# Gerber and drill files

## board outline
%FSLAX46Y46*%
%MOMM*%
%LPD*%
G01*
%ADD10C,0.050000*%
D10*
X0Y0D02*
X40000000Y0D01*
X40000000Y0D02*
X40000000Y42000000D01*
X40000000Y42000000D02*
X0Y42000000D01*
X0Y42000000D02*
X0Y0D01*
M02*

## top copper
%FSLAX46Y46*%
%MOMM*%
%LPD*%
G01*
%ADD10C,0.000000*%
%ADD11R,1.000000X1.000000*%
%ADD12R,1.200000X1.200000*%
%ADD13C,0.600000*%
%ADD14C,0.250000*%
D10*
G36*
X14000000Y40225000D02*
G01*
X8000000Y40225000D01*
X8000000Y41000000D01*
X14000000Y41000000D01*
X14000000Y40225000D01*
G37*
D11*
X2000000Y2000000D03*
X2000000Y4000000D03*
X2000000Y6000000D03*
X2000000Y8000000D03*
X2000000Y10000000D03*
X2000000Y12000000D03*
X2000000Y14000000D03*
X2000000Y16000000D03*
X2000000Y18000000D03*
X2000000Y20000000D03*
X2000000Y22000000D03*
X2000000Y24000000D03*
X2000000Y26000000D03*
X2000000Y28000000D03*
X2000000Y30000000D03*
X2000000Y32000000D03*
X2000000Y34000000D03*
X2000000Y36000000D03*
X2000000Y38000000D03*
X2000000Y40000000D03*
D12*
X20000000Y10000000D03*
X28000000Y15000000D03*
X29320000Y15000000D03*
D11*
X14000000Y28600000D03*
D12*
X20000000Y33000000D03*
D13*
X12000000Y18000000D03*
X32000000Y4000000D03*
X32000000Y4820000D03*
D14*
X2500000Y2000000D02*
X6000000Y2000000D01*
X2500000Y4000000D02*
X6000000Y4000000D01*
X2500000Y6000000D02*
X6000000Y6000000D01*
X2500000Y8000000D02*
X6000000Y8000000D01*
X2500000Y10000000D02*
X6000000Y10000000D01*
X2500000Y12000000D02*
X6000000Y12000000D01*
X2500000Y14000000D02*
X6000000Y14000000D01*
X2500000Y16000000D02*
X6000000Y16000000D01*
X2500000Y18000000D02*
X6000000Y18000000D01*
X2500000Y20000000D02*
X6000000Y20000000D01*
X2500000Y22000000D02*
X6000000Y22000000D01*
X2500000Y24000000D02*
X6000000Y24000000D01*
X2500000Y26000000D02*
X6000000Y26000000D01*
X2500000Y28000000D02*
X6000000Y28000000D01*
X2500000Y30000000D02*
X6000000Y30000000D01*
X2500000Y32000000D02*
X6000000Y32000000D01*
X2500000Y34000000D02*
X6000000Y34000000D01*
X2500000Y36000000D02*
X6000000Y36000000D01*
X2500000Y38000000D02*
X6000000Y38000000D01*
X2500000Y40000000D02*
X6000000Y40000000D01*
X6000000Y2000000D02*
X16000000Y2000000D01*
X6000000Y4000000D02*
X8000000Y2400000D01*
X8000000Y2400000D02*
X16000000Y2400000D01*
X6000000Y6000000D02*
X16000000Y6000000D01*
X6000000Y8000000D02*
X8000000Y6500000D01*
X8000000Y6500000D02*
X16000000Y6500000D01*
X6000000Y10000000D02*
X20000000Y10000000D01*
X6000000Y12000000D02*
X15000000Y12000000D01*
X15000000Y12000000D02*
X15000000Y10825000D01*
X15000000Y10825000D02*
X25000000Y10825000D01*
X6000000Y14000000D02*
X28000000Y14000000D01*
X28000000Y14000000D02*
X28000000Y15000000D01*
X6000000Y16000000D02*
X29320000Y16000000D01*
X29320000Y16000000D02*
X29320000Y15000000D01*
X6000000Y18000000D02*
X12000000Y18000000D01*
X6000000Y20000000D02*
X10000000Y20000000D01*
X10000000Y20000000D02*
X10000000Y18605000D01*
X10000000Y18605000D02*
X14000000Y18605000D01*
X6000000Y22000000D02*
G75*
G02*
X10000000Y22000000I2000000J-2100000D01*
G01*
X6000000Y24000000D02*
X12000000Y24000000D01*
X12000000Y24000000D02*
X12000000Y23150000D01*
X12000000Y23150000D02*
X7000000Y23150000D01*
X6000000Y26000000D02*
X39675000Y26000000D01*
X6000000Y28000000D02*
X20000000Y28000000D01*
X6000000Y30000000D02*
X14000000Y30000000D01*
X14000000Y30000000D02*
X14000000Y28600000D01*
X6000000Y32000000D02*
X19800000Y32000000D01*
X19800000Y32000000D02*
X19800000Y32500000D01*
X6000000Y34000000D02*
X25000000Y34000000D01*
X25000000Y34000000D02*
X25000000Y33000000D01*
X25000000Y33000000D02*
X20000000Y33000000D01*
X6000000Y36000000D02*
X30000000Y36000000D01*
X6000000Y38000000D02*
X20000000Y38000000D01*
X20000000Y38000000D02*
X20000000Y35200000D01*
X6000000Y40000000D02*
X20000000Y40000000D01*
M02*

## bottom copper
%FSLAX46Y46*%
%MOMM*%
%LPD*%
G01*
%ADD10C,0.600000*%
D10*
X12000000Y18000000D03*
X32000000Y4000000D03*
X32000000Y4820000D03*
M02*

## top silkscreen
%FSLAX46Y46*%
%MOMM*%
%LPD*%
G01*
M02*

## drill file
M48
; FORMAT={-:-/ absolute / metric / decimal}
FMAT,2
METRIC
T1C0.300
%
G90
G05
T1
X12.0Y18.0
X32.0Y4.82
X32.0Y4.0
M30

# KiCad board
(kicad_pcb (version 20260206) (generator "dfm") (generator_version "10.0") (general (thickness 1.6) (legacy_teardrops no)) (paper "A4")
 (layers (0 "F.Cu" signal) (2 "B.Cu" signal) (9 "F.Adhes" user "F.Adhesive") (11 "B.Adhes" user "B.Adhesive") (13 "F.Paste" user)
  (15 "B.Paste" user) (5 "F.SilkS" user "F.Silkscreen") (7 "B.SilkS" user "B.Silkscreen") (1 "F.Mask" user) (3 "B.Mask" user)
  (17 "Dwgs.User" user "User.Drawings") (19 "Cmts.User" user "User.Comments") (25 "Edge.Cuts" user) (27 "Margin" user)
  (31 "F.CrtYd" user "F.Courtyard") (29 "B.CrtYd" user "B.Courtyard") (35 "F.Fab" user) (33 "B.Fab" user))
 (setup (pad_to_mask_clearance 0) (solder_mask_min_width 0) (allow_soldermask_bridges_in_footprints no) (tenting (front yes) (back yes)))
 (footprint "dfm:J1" (layer "F.Cu") (at 2 -21 0)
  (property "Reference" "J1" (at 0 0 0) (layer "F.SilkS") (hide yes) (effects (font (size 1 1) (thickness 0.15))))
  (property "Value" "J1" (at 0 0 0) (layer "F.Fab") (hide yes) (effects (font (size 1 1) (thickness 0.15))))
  (pad "1" smd rect (at 0 19 0) (size 1 1) (layers "F.Cu" "F.Mask" "F.Paste") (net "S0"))
  (pad "2" smd rect (at 0 17 0) (size 1 1) (layers "F.Cu" "F.Mask" "F.Paste") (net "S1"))
  (pad "3" smd rect (at 0 15 0) (size 1 1) (layers "F.Cu" "F.Mask" "F.Paste") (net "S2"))
  (pad "4" smd rect (at 0 13 0) (size 1 1) (layers "F.Cu" "F.Mask" "F.Paste") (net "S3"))
  (pad "5" smd rect (at 0 11 0) (size 1 1) (layers "F.Cu" "F.Mask" "F.Paste") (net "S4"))
  (pad "6" smd rect (at 0 9 0) (size 1 1) (layers "F.Cu" "F.Mask" "F.Paste") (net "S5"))
  (pad "7" smd rect (at 0 7 0) (size 1 1) (layers "F.Cu" "F.Mask" "F.Paste") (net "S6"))
  (pad "8" smd rect (at 0 5 0) (size 1 1) (layers "F.Cu" "F.Mask" "F.Paste") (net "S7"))
  (pad "9" smd rect (at 0 3 0) (size 1 1) (layers "F.Cu" "F.Mask" "F.Paste") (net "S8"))
  (pad "10" smd rect (at 0 1 0) (size 1 1) (layers "F.Cu" "F.Mask" "F.Paste") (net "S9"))
  (pad "11" smd rect (at 0 -1 0) (size 1 1) (layers "F.Cu" "F.Mask" "F.Paste") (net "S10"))
  (pad "12" smd rect (at 0 -3 0) (size 1 1) (layers "F.Cu" "F.Mask" "F.Paste") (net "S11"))
  (pad "13" smd rect (at 0 -5 0) (size 1 1) (layers "F.Cu" "F.Mask" "F.Paste") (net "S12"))
  (pad "14" smd rect (at 0 -7 0) (size 1 1) (layers "F.Cu" "F.Mask" "F.Paste") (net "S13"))
  (pad "15" smd rect (at 0 -9 0) (size 1 1) (layers "F.Cu" "F.Mask" "F.Paste") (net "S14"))
  (pad "16" smd rect (at 0 -11 0) (size 1 1) (layers "F.Cu" "F.Mask" "F.Paste") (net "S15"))
  (pad "17" smd rect (at 0 -13 0) (size 1 1) (layers "F.Cu" "F.Mask" "F.Paste") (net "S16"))
  (pad "18" smd rect (at 0 -15 0) (size 1 1) (layers "F.Cu" "F.Mask" "F.Paste") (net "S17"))
  (pad "19" smd rect (at 0 -17 0) (size 1 1) (layers "F.Cu" "F.Mask" "F.Paste") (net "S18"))
  (pad "20" smd rect (at 0 -19 0) (size 1 1) (layers "F.Cu" "F.Mask" "F.Paste") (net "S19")))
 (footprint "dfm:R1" (layer "F.Cu") (at 20 -10 0)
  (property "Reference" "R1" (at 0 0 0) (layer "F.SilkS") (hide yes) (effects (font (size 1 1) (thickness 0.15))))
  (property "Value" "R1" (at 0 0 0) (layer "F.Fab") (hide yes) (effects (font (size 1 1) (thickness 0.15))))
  (pad "1" smd rect (at 0 0 0) (size 1.2 1.2) (layers "F.Cu" "F.Mask" "F.Paste") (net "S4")))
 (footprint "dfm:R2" (layer "F.Cu") (at 28 -15 0)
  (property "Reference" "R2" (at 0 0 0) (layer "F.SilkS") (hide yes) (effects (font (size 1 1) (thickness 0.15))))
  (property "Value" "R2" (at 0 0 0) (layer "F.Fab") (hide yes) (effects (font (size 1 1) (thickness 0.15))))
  (pad "1" smd rect (at 0 0 0) (size 1.2 1.2) (layers "F.Cu" "F.Mask" "F.Paste") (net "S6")))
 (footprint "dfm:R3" (layer "F.Cu") (at 29.32 -15 0)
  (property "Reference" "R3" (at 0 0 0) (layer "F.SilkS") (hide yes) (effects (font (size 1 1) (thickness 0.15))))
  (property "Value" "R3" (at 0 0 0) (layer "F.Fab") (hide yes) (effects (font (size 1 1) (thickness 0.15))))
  (pad "1" smd rect (at 0 0 0) (size 1.2 1.2) (layers "F.Cu" "F.Mask" "F.Paste") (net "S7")))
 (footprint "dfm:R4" (layer "F.Cu") (at 14 -28.6 0)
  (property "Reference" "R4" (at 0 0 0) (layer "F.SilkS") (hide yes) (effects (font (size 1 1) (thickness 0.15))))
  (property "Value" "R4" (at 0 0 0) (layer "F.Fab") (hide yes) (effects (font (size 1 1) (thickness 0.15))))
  (pad "1" smd rect (at 0 0 0) (size 1 1) (layers "F.Cu" "F.Mask" "F.Paste") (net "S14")))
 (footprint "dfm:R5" (layer "F.Cu") (at 20 -33 0)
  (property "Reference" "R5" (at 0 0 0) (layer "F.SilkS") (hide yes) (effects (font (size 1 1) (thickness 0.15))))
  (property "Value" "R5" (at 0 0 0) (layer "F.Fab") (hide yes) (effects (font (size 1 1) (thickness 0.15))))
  (pad "1" smd rect (at 0 0 0) (size 1.2 1.2) (layers "F.Cu" "F.Mask" "F.Paste") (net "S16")))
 (gr_line (start 0 0) (end 40 0) (stroke (width 0.05) (type solid)) (layer "Edge.Cuts"))
 (gr_line (start 40 0) (end 40 -42) (stroke (width 0.05) (type solid)) (layer "Edge.Cuts"))
 (gr_line (start 40 -42) (end 0 -42) (stroke (width 0.05) (type solid)) (layer "Edge.Cuts"))
 (gr_line (start 0 -42) (end 0 0) (stroke (width 0.05) (type solid)) (layer "Edge.Cuts"))
 (segment (start 2.5 -2) (end 6 -2) (width 0.25) (layer "F.Cu") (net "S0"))
 (segment (start 2.5 -4) (end 6 -4) (width 0.25) (layer "F.Cu") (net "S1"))
 (segment (start 2.5 -6) (end 6 -6) (width 0.25) (layer "F.Cu") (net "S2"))
 (segment (start 2.5 -8) (end 6 -8) (width 0.25) (layer "F.Cu") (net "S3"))
 (segment (start 2.5 -10) (end 6 -10) (width 0.25) (layer "F.Cu") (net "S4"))
 (segment (start 2.5 -12) (end 6 -12) (width 0.25) (layer "F.Cu") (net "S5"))
 (segment (start 2.5 -14) (end 6 -14) (width 0.25) (layer "F.Cu") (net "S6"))
 (segment (start 2.5 -16) (end 6 -16) (width 0.25) (layer "F.Cu") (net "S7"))
 (segment (start 2.5 -18) (end 6 -18) (width 0.25) (layer "F.Cu") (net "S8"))
 (segment (start 2.5 -20) (end 6 -20) (width 0.25) (layer "F.Cu") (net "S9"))
 (segment (start 2.5 -22) (end 6 -22) (width 0.25) (layer "F.Cu") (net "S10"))
 (segment (start 2.5 -24) (end 6 -24) (width 0.25) (layer "F.Cu") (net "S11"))
 (segment (start 2.5 -26) (end 6 -26) (width 0.25) (layer "F.Cu") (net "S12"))
 (segment (start 2.5 -28) (end 6 -28) (width 0.25) (layer "F.Cu") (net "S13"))
 (segment (start 2.5 -30) (end 6 -30) (width 0.25) (layer "F.Cu") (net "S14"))
 (segment (start 2.5 -32) (end 6 -32) (width 0.25) (layer "F.Cu") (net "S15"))
 (segment (start 2.5 -34) (end 6 -34) (width 0.25) (layer "F.Cu") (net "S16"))
 (segment (start 2.5 -36) (end 6 -36) (width 0.25) (layer "F.Cu") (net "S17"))
 (segment (start 2.5 -38) (end 6 -38) (width 0.25) (layer "F.Cu") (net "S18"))
 (segment (start 2.5 -40) (end 6 -40) (width 0.25) (layer "F.Cu") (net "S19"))
 (segment (start 6 -2) (end 16 -2) (width 0.25) (layer "F.Cu") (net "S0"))
 (segment (start 6 -4) (end 8 -2.4) (width 0.25) (layer "F.Cu") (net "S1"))
 (segment (start 8 -2.4) (end 16 -2.4) (width 0.25) (layer "F.Cu") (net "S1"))
 (segment (start 6 -6) (end 16 -6) (width 0.25) (layer "F.Cu") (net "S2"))
 (segment (start 6 -8) (end 8 -6.5) (width 0.25) (layer "F.Cu") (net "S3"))
 (segment (start 8 -6.5) (end 16 -6.5) (width 0.25) (layer "F.Cu") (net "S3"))
 (segment (start 6 -10) (end 20 -10) (width 0.25) (layer "F.Cu") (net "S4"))
 (segment (start 6 -12) (end 15 -12) (width 0.25) (layer "F.Cu") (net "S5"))
 (segment (start 15 -12) (end 15 -10.825) (width 0.25) (layer "F.Cu") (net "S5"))
 (segment (start 15 -10.825) (end 25 -10.825) (width 0.25) (layer "F.Cu") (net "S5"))
 (segment (start 6 -14) (end 28 -14) (width 0.25) (layer "F.Cu") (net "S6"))
 (segment (start 28 -14) (end 28 -15) (width 0.25) (layer "F.Cu") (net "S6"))
 (segment (start 6 -16) (end 29.32 -16) (width 0.25) (layer "F.Cu") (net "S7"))
 (segment (start 29.32 -16) (end 29.32 -15) (width 0.25) (layer "F.Cu") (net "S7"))
 (via (at 12 -18) (size 0.6) (drill 0.3) (layers "F.Cu" "B.Cu") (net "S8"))
 (segment (start 6 -18) (end 12 -18) (width 0.25) (layer "F.Cu") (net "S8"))
 (segment (start 6 -20) (end 10 -20) (width 0.25) (layer "F.Cu") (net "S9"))
 (segment (start 10 -20) (end 10 -18.605) (width 0.25) (layer "F.Cu") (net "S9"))
 (segment (start 10 -18.605) (end 14 -18.605) (width 0.25) (layer "F.Cu") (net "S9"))
 (arc (start 6 -22) (mid 8 -22.8) (end 10 -22) (width 0.25) (layer "F.Cu") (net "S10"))
 (segment (start 6 -24) (end 12 -24) (width 0.25) (layer "F.Cu") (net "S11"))
 (segment (start 12 -24) (end 12 -23.15) (width 0.25) (layer "F.Cu") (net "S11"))
 (segment (start 12 -23.15) (end 7 -23.15) (width 0.25) (layer "F.Cu") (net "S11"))
 (segment (start 6 -26) (end 39.675 -26) (width 0.25) (layer "F.Cu") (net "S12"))
 (segment (start 6 -28) (end 20 -28) (width 0.25) (layer "F.Cu") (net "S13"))
 (segment (start 6 -30) (end 14 -30) (width 0.25) (layer "F.Cu") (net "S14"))
 (segment (start 14 -30) (end 14 -28.6) (width 0.25) (layer "F.Cu") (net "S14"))
 (segment (start 6 -32) (end 19.8 -32) (width 0.25) (layer "F.Cu") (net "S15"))
 (segment (start 19.8 -32) (end 19.8 -32.5) (width 0.25) (layer "F.Cu") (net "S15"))
 (segment (start 6 -34) (end 25 -34) (width 0.25) (layer "F.Cu") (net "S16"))
 (segment (start 25 -34) (end 25 -33) (width 0.25) (layer "F.Cu") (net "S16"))
 (segment (start 25 -33) (end 20 -33) (width 0.25) (layer "F.Cu") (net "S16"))
 (segment (start 6 -36) (end 30 -36) (width 0.25) (layer "F.Cu") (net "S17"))
 (segment (start 6 -38) (end 20 -38) (width 0.25) (layer "F.Cu") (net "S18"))
 (segment (start 20 -38) (end 20 -35.2) (width 0.25) (layer "F.Cu") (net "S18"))
 (segment (start 6 -40) (end 20 -40) (width 0.25) (layer "F.Cu") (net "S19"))
 (gr_poly (pts (xy 8 -40.225) (xy 14 -40.225) (xy 14 -41) (xy 8 -41)) (stroke (width 0) (type solid)) (fill yes) (layer "F.Cu"))
 (via (at 32 -4) (size 0.6) (drill 0.3) (layers "F.Cu" "B.Cu") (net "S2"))
 (via (at 32 -4.82) (size 0.6) (drill 0.3) (layers "F.Cu" "B.Cu") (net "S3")))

